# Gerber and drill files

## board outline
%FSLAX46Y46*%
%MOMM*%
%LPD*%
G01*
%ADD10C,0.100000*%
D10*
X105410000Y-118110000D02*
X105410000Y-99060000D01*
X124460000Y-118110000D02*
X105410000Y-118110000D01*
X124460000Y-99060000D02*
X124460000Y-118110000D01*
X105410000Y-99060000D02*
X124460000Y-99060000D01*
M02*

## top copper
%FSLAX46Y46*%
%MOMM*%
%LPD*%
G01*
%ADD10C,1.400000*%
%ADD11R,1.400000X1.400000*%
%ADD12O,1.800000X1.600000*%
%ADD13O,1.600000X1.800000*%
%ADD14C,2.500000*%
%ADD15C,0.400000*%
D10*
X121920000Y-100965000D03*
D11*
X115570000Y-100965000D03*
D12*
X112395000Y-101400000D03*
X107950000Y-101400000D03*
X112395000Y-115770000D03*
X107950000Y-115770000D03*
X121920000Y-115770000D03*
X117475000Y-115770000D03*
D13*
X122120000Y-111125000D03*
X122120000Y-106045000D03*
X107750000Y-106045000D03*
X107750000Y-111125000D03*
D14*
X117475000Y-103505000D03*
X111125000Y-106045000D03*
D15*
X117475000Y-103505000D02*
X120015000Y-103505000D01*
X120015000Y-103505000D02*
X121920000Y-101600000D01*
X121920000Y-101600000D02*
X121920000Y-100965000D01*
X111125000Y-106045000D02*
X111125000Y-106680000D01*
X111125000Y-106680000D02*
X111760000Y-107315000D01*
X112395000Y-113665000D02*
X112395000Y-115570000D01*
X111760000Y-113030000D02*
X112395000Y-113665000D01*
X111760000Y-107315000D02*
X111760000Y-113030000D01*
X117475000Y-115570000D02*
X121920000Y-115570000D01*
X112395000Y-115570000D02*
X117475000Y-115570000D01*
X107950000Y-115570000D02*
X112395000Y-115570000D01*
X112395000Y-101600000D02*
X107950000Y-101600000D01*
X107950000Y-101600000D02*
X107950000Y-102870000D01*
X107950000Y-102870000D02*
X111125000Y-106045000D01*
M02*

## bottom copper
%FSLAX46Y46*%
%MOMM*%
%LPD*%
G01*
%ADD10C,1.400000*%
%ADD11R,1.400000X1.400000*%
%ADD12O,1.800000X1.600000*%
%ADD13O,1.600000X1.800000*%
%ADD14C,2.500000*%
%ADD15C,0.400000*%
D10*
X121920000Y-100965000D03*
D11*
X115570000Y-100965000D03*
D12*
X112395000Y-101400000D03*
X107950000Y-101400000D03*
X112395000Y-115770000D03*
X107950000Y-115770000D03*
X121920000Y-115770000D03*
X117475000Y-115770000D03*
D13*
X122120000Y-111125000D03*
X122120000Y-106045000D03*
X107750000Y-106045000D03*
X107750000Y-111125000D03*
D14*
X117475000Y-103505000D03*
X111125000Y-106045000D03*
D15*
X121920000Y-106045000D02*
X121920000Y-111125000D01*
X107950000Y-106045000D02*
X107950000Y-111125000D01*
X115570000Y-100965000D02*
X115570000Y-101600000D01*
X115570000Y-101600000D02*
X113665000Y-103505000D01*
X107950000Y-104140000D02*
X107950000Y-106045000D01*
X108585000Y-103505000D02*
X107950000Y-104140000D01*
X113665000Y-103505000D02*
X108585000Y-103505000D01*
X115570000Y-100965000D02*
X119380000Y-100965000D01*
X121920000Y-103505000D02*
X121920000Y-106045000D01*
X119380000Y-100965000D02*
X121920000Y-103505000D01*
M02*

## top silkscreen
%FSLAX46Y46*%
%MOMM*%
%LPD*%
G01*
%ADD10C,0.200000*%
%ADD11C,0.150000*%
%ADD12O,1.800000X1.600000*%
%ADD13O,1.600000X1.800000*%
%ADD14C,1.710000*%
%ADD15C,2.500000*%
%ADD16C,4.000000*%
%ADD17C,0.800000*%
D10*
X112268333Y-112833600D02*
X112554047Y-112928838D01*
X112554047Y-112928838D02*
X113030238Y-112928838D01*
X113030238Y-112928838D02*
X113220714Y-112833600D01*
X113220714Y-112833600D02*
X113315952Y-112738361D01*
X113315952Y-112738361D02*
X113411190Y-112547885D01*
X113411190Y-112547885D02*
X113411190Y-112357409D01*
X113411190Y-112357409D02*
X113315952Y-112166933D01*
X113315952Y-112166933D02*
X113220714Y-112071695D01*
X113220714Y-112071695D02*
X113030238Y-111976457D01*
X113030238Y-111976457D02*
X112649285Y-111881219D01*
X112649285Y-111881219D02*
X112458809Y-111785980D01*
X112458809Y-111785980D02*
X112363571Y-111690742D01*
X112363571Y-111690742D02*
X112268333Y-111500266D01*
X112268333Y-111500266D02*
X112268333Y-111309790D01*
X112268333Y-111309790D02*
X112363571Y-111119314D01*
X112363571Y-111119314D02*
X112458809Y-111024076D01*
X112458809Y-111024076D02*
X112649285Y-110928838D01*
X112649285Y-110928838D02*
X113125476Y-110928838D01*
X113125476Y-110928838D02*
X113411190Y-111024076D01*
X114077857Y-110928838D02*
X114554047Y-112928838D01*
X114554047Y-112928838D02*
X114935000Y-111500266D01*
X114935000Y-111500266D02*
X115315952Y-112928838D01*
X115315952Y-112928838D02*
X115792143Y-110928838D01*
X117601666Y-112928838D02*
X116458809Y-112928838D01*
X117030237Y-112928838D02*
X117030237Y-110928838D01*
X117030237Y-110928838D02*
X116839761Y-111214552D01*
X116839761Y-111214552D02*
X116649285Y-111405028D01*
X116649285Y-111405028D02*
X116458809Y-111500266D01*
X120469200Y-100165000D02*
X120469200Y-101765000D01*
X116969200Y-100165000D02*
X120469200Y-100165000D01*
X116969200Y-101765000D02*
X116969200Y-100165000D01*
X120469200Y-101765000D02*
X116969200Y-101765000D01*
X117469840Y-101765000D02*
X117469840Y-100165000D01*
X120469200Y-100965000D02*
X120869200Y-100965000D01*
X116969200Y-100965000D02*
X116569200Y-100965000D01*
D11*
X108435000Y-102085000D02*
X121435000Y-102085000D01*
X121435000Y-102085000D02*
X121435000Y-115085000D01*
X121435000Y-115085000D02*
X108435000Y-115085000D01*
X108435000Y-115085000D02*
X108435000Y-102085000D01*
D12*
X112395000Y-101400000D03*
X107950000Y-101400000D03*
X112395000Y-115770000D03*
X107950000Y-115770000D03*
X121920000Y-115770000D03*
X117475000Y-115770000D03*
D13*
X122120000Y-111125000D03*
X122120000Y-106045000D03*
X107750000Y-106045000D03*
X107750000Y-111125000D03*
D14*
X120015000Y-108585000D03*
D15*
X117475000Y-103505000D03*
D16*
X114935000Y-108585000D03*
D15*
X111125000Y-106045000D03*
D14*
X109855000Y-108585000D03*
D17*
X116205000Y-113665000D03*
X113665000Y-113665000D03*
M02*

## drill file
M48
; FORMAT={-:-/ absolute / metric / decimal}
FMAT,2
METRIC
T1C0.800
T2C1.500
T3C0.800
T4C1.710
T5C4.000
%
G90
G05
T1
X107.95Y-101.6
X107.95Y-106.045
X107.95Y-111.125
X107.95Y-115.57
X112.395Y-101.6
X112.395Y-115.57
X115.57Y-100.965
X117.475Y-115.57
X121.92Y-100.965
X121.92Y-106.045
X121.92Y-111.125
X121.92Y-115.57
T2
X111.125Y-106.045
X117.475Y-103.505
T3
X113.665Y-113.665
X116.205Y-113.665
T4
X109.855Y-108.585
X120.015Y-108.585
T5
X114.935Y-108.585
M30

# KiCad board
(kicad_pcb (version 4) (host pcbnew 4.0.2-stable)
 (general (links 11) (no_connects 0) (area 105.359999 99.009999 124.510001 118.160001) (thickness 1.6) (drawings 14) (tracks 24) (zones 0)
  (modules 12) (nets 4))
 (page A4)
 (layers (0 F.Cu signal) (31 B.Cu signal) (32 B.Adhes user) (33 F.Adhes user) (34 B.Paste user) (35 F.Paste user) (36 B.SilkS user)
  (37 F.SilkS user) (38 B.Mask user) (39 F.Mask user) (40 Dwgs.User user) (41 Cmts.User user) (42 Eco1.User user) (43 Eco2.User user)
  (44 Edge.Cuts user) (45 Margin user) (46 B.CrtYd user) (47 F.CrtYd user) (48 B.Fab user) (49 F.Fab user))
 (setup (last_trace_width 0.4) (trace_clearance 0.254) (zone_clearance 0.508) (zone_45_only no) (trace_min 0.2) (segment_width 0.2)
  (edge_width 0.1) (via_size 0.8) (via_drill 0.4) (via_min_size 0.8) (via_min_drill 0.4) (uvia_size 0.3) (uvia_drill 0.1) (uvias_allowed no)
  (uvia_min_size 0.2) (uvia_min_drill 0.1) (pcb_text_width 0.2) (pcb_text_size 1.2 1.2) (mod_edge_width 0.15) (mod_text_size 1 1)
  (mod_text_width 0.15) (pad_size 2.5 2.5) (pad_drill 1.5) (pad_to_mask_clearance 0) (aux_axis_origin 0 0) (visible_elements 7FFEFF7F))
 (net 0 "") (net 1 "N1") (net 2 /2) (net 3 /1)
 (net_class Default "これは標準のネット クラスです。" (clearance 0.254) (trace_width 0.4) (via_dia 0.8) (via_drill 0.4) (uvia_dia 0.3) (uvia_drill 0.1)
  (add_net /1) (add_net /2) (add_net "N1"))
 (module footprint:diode (layer B.Cu) (at 115.57 100.965)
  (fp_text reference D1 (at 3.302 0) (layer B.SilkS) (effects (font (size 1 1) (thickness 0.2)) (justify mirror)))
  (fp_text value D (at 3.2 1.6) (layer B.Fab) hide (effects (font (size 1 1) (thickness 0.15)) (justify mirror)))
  (fp_line (start 4.8992 -0.8) (end 4.8992 0.8) (layer F.SilkS) (width 0.2))
  (fp_line (start 1.3992 -0.8) (end 4.8992 -0.8) (layer F.SilkS) (width 0.2))
  (fp_line (start 1.3992 0.8) (end 1.3992 -0.8) (layer F.SilkS) (width 0.2))
  (fp_line (start 4.8992 0.8) (end 1.3992 0.8) (layer F.SilkS) (width 0.2))
  (fp_line (start 1.89984 0.8) (end 1.89984 -0.8) (layer F.SilkS) (width 0.2))
  (fp_line (start 4.8992 0) (end 5.2992 0) (layer F.SilkS) (width 0.2))
  (fp_line (start 1.3992 0) (end 0.9992 0) (layer F.SilkS) (width 0.2))
  (pad 2 thru_hole circle (at 6.35 0) (size 1.4 1.4) (drill 0.8) (layers *.Cu *.Mask B.SilkS) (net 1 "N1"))
  (pad 1 thru_hole rect (at 0 0) (size 1.4 1.4) (drill 0.8) (layers *.Cu *.Mask B.SilkS) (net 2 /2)))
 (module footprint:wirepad (layer F.Cu) (at 112.395 101.6 180)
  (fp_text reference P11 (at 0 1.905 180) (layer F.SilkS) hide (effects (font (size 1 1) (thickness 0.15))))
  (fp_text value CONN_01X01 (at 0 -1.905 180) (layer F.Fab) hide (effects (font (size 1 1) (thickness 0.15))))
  (pad 1 thru_hole oval (at 0 0 180) (size 1.8 1.6) (drill 0.8 (offset 0 0.2)) (layers *.Cu *.Mask F.SilkS) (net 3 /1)))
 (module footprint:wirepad (layer F.Cu) (at 107.95 101.6 180)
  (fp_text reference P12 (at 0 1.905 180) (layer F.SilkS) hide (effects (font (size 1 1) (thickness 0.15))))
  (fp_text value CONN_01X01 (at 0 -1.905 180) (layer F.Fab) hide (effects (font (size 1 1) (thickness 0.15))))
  (pad 1 thru_hole oval (at 0 0 180) (size 1.8 1.6) (drill 0.8 (offset 0 0.2)) (layers *.Cu *.Mask F.SilkS) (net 3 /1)))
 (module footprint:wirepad (layer F.Cu) (at 112.395 115.57)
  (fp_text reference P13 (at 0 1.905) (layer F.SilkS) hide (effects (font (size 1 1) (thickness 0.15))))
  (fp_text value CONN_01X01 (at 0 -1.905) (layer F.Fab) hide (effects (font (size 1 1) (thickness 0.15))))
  (pad 1 thru_hole oval (at 0 0) (size 1.8 1.6) (drill 0.8 (offset 0 0.2)) (layers *.Cu *.Mask F.SilkS) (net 3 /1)))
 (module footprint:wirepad (layer F.Cu) (at 107.95 115.57)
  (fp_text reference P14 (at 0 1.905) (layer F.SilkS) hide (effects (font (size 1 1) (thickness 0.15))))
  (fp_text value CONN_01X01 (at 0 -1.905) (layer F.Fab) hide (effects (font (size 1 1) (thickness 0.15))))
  (pad 1 thru_hole oval (at 0 0) (size 1.8 1.6) (drill 0.8 (offset 0 0.2)) (layers *.Cu *.Mask F.SilkS) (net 3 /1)))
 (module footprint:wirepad (layer F.Cu) (at 121.92 115.57)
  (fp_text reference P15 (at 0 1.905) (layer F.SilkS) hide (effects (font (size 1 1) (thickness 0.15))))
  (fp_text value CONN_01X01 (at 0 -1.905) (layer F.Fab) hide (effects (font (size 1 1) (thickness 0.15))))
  (pad 1 thru_hole oval (at 0 0) (size 1.8 1.6) (drill 0.8 (offset 0 0.2)) (layers *.Cu *.Mask F.SilkS) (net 3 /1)))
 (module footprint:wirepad (layer F.Cu) (at 117.475 115.57)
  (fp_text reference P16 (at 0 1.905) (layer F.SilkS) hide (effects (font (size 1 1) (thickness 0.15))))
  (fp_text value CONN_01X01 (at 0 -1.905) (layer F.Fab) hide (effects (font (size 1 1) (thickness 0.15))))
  (pad 1 thru_hole oval (at 0 0) (size 1.8 1.6) (drill 0.8 (offset 0 0.2)) (layers *.Cu *.Mask F.SilkS) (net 3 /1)))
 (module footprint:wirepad (layer F.Cu) (at 121.92 111.125 90)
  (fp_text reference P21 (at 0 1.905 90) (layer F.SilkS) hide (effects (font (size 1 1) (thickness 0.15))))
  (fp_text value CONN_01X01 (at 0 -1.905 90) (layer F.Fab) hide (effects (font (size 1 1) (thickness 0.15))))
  (pad 1 thru_hole oval (at 0 0 90) (size 1.8 1.6) (drill 0.8 (offset 0 0.2)) (layers *.Cu *.Mask F.SilkS) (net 2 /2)))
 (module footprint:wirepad (layer F.Cu) (at 121.92 106.045 90)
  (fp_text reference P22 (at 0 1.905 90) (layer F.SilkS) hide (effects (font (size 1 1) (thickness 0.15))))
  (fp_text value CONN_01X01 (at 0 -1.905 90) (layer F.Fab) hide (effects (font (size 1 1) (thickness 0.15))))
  (pad 1 thru_hole oval (at 0 0 90) (size 1.8 1.6) (drill 0.8 (offset 0 0.2)) (layers *.Cu *.Mask F.SilkS) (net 2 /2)))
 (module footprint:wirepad (layer F.Cu) (at 107.95 106.045 270)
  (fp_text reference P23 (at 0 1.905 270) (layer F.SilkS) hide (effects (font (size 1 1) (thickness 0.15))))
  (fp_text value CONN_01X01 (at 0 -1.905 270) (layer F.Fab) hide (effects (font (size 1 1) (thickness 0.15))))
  (pad 1 thru_hole oval (at 0 0 270) (size 1.8 1.6) (drill 0.8 (offset 0 0.2)) (layers *.Cu *.Mask F.SilkS) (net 2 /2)))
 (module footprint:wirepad (layer F.Cu) (at 107.95 111.125 270)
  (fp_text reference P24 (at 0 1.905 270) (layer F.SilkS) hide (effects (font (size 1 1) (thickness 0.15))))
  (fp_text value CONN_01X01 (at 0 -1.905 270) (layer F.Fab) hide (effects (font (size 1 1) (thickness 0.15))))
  (pad 1 thru_hole oval (at 0 0 270) (size 1.8 1.6) (drill 0.8 (offset 0 0.2)) (layers *.Cu *.Mask F.SilkS) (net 2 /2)))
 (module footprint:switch (layer F.Cu) (at 114.935 108.585)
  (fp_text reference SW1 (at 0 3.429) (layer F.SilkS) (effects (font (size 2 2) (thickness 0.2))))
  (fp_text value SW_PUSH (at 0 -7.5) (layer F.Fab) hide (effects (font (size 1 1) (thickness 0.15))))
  (fp_line (start -6.5 -6.5) (end 6.5 -6.5) (layer F.SilkS) (width 0.15))
  (fp_line (start 6.5 -6.5) (end 6.5 6.5) (layer F.SilkS) (width 0.15))
  (fp_line (start 6.5 6.5) (end -6.5 6.5) (layer F.SilkS) (width 0.15))
  (fp_line (start -6.5 6.5) (end -6.5 -6.5) (layer F.SilkS) (width 0.15))
  (pad "" np_thru_hole circle (at 5.08 0) (size 1.71 1.71) (drill 1.71) (layers *.Cu *.Mask F.SilkS))
  (pad 2 thru_hole circle (at 2.54 -5.08) (size 2.5 2.5) (drill 1.5) (layers *.Cu *.Mask F.SilkS) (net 1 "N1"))
  (pad "" np_thru_hole circle (at 0 0) (size 4 4) (drill 4) (layers *.Cu *.Mask F.SilkS))
  (pad 1 thru_hole circle (at -3.81 -2.54) (size 2.5 2.5) (drill 1.5) (layers *.Cu *.Mask F.SilkS) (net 3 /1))
  (pad "" np_thru_hole circle (at -5.08 0) (size 1.71 1.71) (drill 1.71) (layers *.Cu *.Mask F.SilkS))
  (pad "" np_thru_hole circle (at 1.27 5.08) (size 0.8 0.8) (drill 0.8) (layers *.Cu *.Mask F.SilkS))
  (pad "" np_thru_hole circle (at -1.27 5.08) (size 0.8 0.8) (drill 0.8) (layers *.Cu *.Mask F.SilkS)))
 (gr_line (start 105.41 118.11) (end 105.41 99.06) (angle 90) (layer Edge.Cuts) (width 0.1))
 (gr_line (start 124.46 118.11) (end 105.41 118.11) (angle 90) (layer Edge.Cuts) (width 0.1))
 (gr_line (start 124.46 99.06) (end 124.46 118.11) (angle 90) (layer Edge.Cuts) (width 0.1))
 (gr_line (start 105.41 99.06) (end 124.46 99.06) (angle 90) (layer Edge.Cuts) (width 0.1))
 (segment (start 117.475 103.505) (end 120.015 103.505) (width 0.4) (layer F.Cu) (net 1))
 (segment (start 120.015 103.505) (end 121.92 101.6) (width 0.4) (layer F.Cu) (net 1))
 (segment (start 121.92 101.6) (end 121.92 100.965) (width 0.4) (layer F.Cu) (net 1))
 (segment (start 121.92 106.045) (end 121.92 111.125) (width 0.4) (layer B.Cu) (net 2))
 (segment (start 107.95 106.045) (end 107.95 111.125) (width 0.4) (layer B.Cu) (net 2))
 (segment (start 115.57 100.965) (end 115.57 101.6) (width 0.4) (layer B.Cu) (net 2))
 (segment (start 115.57 101.6) (end 113.665 103.505) (width 0.4) (layer B.Cu) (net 2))
 (segment (start 107.95 104.14) (end 107.95 106.045) (width 0.4) (layer B.Cu) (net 2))
 (segment (start 108.585 103.505) (end 107.95 104.14) (width 0.4) (layer B.Cu) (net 2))
 (segment (start 113.665 103.505) (end 108.585 103.505) (width 0.4) (layer B.Cu) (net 2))
 (segment (start 115.57 100.965) (end 119.38 100.965) (width 0.4) (layer B.Cu) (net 2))
 (segment (start 121.92 103.505) (end 121.92 106.045) (width 0.4) (layer B.Cu) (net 2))
 (segment (start 119.38 100.965) (end 121.92 103.505) (width 0.4) (layer B.Cu) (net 2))
 (segment (start 111.125 106.045) (end 111.125 106.68) (width 0.4) (layer F.Cu) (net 3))
 (segment (start 111.125 106.68) (end 111.76 107.315) (width 0.4) (layer F.Cu) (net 3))
 (segment (start 112.395 113.665) (end 112.395 115.57) (width 0.4) (layer F.Cu) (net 3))
 (segment (start 111.76 113.03) (end 112.395 113.665) (width 0.4) (layer F.Cu) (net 3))
 (segment (start 111.76 107.315) (end 111.76 113.03) (width 0.4) (layer F.Cu) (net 3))
 (segment (start 117.475 115.57) (end 121.92 115.57) (width 0.4) (layer F.Cu) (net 3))
 (segment (start 112.395 115.57) (end 117.475 115.57) (width 0.4) (layer F.Cu) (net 3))
 (segment (start 107.95 115.57) (end 112.395 115.57) (width 0.4) (layer F.Cu) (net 3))
 (segment (start 112.395 101.6) (end 107.95 101.6) (width 0.4) (layer F.Cu) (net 3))
 (segment (start 107.95 101.6) (end 107.95 102.87) (width 0.4) (layer F.Cu) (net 3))
 (segment (start 107.95 102.87) (end 111.125 106.045) (width 0.4) (layer F.Cu) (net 3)))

